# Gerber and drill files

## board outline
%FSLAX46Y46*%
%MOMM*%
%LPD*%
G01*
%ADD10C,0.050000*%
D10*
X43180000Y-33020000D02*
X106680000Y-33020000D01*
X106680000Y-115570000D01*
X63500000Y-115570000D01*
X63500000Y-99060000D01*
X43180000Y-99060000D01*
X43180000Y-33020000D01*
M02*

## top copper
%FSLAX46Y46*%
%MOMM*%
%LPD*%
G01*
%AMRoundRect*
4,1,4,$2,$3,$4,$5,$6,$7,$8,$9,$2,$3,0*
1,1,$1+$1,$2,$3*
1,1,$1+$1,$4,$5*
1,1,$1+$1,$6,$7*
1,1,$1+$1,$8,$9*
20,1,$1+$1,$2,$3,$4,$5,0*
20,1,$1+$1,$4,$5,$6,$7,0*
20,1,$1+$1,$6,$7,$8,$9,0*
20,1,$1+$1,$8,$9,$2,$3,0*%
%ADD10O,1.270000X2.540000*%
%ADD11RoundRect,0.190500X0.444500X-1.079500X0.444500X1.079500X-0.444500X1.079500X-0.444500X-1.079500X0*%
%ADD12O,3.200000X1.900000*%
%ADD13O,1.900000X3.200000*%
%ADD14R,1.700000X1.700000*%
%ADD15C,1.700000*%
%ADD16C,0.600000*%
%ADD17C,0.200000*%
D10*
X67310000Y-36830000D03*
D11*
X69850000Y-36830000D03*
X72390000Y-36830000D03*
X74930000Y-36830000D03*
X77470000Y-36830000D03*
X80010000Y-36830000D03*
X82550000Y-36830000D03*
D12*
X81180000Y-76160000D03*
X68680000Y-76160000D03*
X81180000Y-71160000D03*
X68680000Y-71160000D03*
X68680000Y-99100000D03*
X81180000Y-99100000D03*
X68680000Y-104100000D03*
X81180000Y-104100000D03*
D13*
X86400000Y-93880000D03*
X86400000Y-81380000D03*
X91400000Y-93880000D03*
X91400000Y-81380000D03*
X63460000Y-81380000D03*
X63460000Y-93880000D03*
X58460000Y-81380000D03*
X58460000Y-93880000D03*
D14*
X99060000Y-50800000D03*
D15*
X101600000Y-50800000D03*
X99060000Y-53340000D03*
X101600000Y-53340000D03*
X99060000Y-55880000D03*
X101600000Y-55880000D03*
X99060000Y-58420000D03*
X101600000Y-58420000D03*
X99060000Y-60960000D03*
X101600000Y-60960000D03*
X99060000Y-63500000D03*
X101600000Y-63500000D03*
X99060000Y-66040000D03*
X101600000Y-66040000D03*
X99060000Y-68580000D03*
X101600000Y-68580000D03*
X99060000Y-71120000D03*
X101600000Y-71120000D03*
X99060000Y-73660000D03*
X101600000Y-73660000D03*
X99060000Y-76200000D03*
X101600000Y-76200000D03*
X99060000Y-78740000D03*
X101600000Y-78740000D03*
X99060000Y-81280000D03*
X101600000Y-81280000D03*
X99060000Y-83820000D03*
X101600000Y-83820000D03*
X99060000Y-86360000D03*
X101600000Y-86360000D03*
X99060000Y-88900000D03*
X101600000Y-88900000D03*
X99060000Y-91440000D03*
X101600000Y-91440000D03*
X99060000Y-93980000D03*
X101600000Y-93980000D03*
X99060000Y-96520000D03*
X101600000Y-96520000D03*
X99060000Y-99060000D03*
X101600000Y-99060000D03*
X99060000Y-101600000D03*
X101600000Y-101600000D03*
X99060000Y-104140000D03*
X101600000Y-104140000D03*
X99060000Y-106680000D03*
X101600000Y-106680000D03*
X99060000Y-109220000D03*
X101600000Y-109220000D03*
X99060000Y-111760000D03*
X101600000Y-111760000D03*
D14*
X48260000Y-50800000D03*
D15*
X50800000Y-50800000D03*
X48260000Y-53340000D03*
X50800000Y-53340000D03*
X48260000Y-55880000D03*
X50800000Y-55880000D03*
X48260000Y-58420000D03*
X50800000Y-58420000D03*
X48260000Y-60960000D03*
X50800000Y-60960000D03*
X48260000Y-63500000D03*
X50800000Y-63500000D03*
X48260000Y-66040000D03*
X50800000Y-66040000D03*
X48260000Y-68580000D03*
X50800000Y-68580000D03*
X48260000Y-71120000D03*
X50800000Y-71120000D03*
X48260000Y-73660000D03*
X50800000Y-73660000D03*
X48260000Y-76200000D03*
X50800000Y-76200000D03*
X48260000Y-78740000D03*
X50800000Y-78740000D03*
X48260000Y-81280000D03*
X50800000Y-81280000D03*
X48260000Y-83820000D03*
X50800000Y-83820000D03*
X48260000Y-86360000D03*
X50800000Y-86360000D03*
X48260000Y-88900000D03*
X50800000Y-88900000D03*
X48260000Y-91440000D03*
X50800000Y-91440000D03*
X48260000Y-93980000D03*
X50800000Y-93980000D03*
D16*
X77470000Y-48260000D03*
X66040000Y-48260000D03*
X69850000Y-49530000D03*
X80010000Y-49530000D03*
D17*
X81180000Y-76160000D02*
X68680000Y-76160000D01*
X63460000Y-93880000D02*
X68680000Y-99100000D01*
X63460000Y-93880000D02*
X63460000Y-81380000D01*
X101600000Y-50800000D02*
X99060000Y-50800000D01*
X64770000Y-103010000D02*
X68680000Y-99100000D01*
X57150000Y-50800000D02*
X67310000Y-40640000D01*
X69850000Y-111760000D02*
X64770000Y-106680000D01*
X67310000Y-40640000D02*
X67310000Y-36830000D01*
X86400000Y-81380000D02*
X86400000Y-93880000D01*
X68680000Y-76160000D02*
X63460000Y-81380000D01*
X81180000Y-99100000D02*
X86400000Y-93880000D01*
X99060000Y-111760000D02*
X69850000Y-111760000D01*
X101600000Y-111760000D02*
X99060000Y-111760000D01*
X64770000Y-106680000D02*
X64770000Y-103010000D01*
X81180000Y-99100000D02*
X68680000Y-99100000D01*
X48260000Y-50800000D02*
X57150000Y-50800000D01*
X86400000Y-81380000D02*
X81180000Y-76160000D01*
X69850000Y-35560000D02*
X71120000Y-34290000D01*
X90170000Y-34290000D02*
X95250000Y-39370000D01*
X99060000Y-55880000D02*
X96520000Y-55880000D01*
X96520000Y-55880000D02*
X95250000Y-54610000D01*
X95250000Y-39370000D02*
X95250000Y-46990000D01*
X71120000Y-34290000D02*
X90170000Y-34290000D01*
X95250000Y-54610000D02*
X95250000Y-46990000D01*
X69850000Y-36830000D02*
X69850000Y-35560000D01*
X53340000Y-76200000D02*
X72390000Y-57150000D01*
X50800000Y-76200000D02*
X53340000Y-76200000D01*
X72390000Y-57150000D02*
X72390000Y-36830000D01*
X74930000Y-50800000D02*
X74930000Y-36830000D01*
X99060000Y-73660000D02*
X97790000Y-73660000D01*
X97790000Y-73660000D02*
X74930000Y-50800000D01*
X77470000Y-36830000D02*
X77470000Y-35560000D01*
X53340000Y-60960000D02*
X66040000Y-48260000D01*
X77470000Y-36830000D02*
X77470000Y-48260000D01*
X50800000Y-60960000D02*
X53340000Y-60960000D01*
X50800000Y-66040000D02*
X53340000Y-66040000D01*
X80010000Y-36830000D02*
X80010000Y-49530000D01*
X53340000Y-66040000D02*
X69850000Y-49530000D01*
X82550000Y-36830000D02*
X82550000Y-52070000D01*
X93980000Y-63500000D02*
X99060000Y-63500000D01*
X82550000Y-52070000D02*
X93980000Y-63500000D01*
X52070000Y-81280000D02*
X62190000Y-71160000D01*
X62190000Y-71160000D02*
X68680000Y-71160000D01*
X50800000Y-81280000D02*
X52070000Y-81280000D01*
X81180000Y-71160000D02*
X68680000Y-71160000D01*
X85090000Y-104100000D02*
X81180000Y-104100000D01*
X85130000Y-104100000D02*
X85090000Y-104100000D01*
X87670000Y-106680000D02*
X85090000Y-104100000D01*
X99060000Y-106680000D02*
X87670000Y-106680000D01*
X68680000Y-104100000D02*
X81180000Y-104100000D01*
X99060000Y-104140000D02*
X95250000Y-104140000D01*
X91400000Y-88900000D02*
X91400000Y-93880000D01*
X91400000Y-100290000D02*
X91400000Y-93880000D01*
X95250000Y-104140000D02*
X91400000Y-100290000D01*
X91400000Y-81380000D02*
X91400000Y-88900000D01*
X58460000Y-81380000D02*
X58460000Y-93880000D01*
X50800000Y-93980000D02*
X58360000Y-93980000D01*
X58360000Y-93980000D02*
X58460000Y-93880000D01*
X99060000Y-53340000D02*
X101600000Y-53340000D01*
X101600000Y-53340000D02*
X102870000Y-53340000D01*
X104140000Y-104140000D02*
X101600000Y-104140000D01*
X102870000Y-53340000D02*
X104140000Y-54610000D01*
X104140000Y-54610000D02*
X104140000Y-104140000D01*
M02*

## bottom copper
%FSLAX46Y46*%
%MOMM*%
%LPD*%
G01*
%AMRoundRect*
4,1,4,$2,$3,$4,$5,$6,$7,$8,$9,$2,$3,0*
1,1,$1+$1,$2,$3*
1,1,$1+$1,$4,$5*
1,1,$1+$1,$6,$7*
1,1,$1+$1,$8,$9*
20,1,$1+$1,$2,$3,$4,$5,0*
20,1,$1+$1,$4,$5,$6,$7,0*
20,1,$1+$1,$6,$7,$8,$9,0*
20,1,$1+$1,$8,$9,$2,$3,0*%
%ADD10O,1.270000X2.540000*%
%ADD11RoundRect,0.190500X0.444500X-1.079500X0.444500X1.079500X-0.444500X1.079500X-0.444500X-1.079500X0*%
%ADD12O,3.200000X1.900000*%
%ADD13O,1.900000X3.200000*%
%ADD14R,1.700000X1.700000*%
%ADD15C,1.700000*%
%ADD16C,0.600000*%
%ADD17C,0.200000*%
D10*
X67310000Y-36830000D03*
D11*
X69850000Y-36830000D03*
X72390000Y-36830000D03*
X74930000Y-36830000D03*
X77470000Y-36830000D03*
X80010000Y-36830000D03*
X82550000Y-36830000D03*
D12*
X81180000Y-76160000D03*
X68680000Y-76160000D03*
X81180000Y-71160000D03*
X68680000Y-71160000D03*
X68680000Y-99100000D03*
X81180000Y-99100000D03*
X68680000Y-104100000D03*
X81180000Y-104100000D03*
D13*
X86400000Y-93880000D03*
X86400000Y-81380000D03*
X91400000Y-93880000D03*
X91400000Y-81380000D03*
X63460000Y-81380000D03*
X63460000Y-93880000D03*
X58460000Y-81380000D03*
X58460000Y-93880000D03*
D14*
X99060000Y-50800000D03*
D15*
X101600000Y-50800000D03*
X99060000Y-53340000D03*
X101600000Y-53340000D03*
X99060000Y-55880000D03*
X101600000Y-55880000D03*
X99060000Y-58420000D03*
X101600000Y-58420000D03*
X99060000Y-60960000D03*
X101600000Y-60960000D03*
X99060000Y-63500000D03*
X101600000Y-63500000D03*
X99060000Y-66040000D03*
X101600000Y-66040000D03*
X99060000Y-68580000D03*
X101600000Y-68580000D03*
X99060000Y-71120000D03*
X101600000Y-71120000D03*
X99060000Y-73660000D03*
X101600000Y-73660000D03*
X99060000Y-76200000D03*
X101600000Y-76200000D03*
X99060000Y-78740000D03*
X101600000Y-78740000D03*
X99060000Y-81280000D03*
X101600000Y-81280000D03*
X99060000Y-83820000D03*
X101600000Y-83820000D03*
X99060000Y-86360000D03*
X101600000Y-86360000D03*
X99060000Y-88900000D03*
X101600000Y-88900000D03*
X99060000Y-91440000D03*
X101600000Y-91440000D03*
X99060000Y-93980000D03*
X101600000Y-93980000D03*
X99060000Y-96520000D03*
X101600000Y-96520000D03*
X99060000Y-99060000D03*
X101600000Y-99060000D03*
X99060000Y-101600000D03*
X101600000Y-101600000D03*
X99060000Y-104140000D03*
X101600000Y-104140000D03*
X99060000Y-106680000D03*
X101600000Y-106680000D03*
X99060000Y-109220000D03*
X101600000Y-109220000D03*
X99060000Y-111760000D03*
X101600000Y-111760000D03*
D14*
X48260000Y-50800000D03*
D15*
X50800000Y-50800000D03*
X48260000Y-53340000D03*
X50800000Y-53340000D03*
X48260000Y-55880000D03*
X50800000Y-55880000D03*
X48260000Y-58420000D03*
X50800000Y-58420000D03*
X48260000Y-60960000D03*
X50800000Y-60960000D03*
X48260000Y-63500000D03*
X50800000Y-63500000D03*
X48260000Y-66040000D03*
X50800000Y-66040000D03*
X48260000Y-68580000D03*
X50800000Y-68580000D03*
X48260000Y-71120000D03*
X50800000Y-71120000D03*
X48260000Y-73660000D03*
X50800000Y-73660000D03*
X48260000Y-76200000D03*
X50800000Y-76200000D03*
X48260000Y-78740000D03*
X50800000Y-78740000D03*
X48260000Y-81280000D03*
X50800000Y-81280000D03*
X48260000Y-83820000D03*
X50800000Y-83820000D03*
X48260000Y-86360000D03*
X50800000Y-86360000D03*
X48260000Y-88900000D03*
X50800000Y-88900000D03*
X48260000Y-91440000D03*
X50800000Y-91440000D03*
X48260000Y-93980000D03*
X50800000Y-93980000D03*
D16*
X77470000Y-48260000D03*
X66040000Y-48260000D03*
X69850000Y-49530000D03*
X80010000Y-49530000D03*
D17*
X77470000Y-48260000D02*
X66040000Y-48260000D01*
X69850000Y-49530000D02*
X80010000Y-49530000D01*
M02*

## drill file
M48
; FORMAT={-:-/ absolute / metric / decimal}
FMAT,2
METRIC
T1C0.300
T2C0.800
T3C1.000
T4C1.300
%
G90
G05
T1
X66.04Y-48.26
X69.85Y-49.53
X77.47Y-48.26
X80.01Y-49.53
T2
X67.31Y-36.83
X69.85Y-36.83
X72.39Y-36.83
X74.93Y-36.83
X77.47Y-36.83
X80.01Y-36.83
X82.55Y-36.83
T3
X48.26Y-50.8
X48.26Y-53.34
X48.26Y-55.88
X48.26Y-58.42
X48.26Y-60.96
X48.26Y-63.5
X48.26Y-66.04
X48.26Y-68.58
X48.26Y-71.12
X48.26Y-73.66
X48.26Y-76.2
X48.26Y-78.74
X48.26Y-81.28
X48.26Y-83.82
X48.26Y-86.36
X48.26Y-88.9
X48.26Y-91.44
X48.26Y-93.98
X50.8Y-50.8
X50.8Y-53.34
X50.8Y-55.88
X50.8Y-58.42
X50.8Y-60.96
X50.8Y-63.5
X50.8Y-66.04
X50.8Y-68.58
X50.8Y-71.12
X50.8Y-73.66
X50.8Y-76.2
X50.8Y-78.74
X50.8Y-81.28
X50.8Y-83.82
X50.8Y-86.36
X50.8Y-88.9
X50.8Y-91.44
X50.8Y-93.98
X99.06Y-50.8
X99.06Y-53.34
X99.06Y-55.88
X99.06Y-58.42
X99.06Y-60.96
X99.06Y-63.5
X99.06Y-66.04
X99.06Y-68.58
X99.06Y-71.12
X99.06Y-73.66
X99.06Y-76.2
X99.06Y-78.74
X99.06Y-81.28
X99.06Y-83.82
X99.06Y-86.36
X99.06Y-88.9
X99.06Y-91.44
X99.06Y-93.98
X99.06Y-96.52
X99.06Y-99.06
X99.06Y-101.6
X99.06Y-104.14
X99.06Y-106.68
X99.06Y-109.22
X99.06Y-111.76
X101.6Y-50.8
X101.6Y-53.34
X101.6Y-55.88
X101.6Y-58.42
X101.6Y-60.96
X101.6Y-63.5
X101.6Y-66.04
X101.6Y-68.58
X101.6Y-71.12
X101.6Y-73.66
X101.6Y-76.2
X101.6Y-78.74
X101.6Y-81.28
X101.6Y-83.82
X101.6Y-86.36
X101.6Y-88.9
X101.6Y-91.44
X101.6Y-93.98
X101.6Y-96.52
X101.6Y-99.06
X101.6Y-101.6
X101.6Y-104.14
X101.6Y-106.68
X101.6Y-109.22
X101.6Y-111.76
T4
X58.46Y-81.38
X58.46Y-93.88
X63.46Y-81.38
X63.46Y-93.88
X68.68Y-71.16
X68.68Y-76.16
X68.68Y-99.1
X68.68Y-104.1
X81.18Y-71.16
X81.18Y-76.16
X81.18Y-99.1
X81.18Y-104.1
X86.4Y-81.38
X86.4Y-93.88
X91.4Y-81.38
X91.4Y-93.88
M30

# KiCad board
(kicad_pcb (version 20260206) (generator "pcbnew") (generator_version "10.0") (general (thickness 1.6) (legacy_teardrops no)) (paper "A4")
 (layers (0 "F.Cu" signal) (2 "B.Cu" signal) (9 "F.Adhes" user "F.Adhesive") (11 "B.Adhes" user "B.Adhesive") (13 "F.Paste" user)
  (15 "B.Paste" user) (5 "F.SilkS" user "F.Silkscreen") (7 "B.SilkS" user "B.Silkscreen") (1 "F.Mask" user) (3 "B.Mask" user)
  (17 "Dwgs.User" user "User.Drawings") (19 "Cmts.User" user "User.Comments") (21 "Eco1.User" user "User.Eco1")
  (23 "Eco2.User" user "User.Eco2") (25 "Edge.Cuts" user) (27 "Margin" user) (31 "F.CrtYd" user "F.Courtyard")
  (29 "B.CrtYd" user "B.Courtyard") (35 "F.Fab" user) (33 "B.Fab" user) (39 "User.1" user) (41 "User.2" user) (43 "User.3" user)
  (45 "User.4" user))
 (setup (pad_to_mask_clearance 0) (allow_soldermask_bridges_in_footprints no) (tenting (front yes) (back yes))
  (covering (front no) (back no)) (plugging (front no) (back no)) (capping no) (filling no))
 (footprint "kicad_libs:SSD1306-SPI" (layer "F.Cu") (at 74.93 46.99)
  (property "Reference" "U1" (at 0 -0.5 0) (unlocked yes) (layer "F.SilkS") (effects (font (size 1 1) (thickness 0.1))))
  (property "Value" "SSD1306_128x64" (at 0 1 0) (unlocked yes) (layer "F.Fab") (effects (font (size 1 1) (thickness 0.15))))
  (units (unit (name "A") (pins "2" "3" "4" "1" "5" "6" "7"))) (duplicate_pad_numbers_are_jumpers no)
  (pad "1" thru_hole oval (at -7.62 -10.16 90) (size 2.54 1.27) (drill 0.8) (layers "*.Cu" "*.Mask") (remove_unused_layers no) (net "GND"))
  (pad "2" thru_hole roundrect (at -5.08 -10.16 90) (size 2.54 1.27) (drill 0.8) (layers "*.Cu" "*.Mask") (remove_unused_layers no)
   (roundrect_rratio 0.15) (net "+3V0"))
  (pad "3" thru_hole roundrect (at -2.54 -10.16 90) (size 2.54 1.27) (drill 0.8) (layers "*.Cu" "*.Mask") (remove_unused_layers no)
   (roundrect_rratio 0.15) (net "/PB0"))
  (pad "4" thru_hole roundrect (at 0 -10.16 90) (size 2.54 1.27) (drill 0.8) (layers "*.Cu" "*.Mask") (remove_unused_layers no)
   (roundrect_rratio 0.15) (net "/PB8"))
  (pad "5" thru_hole roundrect (at 2.54 -10.16 90) (size 2.54 1.27) (drill 0.8) (layers "*.Cu" "*.Mask") (remove_unused_layers no)
   (roundrect_rratio 0.15) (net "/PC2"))
  (pad "6" thru_hole roundrect (at 5.08 -10.16 90) (size 2.54 1.27) (drill 0.8) (layers "*.Cu" "*.Mask") (remove_unused_layers no)
   (roundrect_rratio 0.15) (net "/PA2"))
  (pad "7" thru_hole roundrect (at 7.62 -10.16 90) (size 2.54 1.27) (drill 0.8) (layers "*.Cu" "*.Mask") (remove_unused_layers no)
   (roundrect_rratio 0.15) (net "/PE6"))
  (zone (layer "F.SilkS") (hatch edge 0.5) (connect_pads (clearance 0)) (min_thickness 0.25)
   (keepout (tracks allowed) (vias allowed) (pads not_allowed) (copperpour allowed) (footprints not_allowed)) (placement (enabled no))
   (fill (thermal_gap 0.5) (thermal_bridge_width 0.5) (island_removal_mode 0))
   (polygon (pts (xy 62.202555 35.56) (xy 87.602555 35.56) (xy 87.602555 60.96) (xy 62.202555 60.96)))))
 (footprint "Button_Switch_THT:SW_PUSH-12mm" (layer "F.Cu") (at 81.18 76.16 180)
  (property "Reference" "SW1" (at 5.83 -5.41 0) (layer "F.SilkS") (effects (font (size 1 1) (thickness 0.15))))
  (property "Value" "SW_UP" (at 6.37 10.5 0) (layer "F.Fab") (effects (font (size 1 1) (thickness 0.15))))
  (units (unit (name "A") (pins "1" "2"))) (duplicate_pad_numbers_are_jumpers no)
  (pad "1" thru_hole oval (at 0 0 180) (size 3.2 1.9) (drill 1.3) (layers "*.Cu" "*.Mask") (remove_unused_layers no) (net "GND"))
  (pad "1" thru_hole oval (at 12.5 0 180) (size 3.2 1.9) (drill 1.3) (layers "*.Cu" "*.Mask") (remove_unused_layers no) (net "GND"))
  (pad "2" thru_hole oval (at 0 5 180) (size 3.2 1.9) (drill 1.3) (layers "*.Cu" "*.Mask") (remove_unused_layers no) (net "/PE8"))
  (pad "2" thru_hole oval (at 12.5 5 180) (size 3.2 1.9) (drill 1.3) (layers "*.Cu" "*.Mask") (remove_unused_layers no) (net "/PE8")))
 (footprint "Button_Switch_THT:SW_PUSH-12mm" (layer "F.Cu") (at 68.68 99.1)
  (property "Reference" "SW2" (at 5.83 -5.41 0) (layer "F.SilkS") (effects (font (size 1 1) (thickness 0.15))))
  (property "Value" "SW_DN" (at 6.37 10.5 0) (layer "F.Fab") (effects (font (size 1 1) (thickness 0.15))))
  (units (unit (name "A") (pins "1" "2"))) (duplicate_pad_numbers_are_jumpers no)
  (pad "1" thru_hole oval (at 0 0) (size 3.2 1.9) (drill 1.3) (layers "*.Cu" "*.Mask") (remove_unused_layers no) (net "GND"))
  (pad "1" thru_hole oval (at 12.5 0) (size 3.2 1.9) (drill 1.3) (layers "*.Cu" "*.Mask") (remove_unused_layers no) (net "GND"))
  (pad "2" thru_hole oval (at 0 5) (size 3.2 1.9) (drill 1.3) (layers "*.Cu" "*.Mask") (remove_unused_layers no) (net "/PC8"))
  (pad "2" thru_hole oval (at 12.5 5) (size 3.2 1.9) (drill 1.3) (layers "*.Cu" "*.Mask") (remove_unused_layers no) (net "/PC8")))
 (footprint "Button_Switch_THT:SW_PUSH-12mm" (layer "F.Cu") (at 86.4 93.88 90)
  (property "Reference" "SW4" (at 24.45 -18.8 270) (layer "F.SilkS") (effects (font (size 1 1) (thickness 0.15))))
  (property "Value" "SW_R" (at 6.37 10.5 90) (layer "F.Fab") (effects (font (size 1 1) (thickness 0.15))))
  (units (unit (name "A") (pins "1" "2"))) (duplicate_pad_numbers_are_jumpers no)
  (pad "1" thru_hole oval (at 0 0 90) (size 3.2 1.9) (drill 1.3) (layers "*.Cu" "*.Mask") (remove_unused_layers no) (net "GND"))
  (pad "1" thru_hole oval (at 12.5 0 90) (size 3.2 1.9) (drill 1.3) (layers "*.Cu" "*.Mask") (remove_unused_layers no) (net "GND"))
  (pad "2" thru_hole oval (at 0 5 90) (size 3.2 1.9) (drill 1.3) (layers "*.Cu" "*.Mask") (remove_unused_layers no) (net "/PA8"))
  (pad "2" thru_hole oval (at 12.5 5 90) (size 3.2 1.9) (drill 1.3) (layers "*.Cu" "*.Mask") (remove_unused_layers no) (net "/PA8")))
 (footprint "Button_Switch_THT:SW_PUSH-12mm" (layer "F.Cu") (at 63.46 81.38 -90)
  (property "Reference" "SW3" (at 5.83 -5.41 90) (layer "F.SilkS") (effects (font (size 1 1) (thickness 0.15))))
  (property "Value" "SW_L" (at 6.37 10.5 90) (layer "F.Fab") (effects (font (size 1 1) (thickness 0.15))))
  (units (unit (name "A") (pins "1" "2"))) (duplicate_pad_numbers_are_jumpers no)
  (pad "1" thru_hole oval (at 0 0 270) (size 3.2 1.9) (drill 1.3) (layers "*.Cu" "*.Mask") (remove_unused_layers no) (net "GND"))
  (pad "1" thru_hole oval (at 12.5 0 270) (size 3.2 1.9) (drill 1.3) (layers "*.Cu" "*.Mask") (remove_unused_layers no) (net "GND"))
  (pad "2" thru_hole oval (at 0 5 270) (size 3.2 1.9) (drill 1.3) (layers "*.Cu" "*.Mask") (remove_unused_layers no) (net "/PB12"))
  (pad "2" thru_hole oval (at 12.5 5 270) (size 3.2 1.9) (drill 1.3) (layers "*.Cu" "*.Mask") (remove_unused_layers no) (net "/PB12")))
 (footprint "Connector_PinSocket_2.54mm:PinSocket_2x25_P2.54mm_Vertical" (layer "B.Cu") (at 99.06 50.8 180)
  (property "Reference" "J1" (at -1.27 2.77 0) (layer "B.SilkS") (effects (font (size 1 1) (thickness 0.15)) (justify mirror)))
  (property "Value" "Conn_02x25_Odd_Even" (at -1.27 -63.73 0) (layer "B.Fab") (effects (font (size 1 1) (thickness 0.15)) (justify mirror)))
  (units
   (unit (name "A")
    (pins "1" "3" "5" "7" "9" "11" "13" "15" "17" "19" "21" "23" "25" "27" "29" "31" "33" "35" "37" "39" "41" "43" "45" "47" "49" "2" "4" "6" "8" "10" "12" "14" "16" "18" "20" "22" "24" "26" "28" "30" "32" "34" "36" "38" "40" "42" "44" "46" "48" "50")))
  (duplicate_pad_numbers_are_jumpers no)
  (pad "1" thru_hole rect (at 0 0 180) (size 1.7 1.7) (drill 1) (layers "*.Cu" "*.Mask") (remove_unused_layers no) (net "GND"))
  (pad "2" thru_hole circle (at -2.54 0 180) (size 1.7 1.7) (drill 1) (layers "*.Cu" "*.Mask") (remove_unused_layers no) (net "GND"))
  (pad "3" thru_hole circle (at 0 -2.54 180) (size 1.7 1.7) (drill 1) (layers "*.Cu" "*.Mask") (remove_unused_layers no) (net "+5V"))
  (pad "4" thru_hole circle (at -2.54 -2.54 180) (size 1.7 1.7) (drill 1) (layers "*.Cu" "*.Mask") (remove_unused_layers no) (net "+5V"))
  (pad "5" thru_hole circle (at 0 -5.08 180) (size 1.7 1.7) (drill 1) (layers "*.Cu" "*.Mask") (remove_unused_layers no) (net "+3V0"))
  (pad "6" thru_hole circle (at -2.54 -5.08 180) (size 1.7 1.7) (drill 1) (layers "*.Cu" "*.Mask") (remove_unused_layers no) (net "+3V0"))
  (pad "7" thru_hole circle (at 0 -7.62 180) (size 1.7 1.7) (drill 1) (layers "*.Cu" "*.Mask") (remove_unused_layers no)
   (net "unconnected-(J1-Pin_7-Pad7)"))
  (pad "8" thru_hole circle (at -2.54 -7.62 180) (size 1.7 1.7) (drill 1) (layers "*.Cu" "*.Mask") (remove_unused_layers no)
   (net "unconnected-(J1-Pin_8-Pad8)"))
  (pad "9" thru_hole circle (at 0 -10.16 180) (size 1.7 1.7) (drill 1) (layers "*.Cu" "*.Mask") (remove_unused_layers no)
   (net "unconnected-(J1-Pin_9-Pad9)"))
  (pad "10" thru_hole circle (at -2.54 -10.16 180) (size 1.7 1.7) (drill 1) (layers "*.Cu" "*.Mask") (remove_unused_layers no)
   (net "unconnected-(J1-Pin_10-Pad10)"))
  (pad "11" thru_hole circle (at 0 -12.7 180) (size 1.7 1.7) (drill 1) (layers "*.Cu" "*.Mask") (remove_unused_layers no) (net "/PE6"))
  (pad "12" thru_hole circle (at -2.54 -12.7 180) (size 1.7 1.7) (drill 1) (layers "*.Cu" "*.Mask") (remove_unused_layers no)
   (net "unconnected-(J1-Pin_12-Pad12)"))
  (pad "13" thru_hole circle (at 0 -15.24 180) (size 1.7 1.7) (drill 1) (layers "*.Cu" "*.Mask") (remove_unused_layers no)
   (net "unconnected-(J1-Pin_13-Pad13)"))
  (pad "14" thru_hole circle (at -2.54 -15.24 180) (size 1.7 1.7) (drill 1) (layers "*.Cu" "*.Mask") (remove_unused_layers no)
   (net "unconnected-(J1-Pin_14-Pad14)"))
  (pad "15" thru_hole circle (at 0 -17.78 180) (size 1.7 1.7) (drill 1) (layers "*.Cu" "*.Mask") (remove_unused_layers no)
   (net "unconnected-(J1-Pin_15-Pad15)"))
  (pad "16" thru_hole circle (at -2.54 -17.78 180) (size 1.7 1.7) (drill 1) (layers "*.Cu" "*.Mask") (remove_unused_layers no)
   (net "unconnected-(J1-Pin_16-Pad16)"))
  (pad "17" thru_hole circle (at 0 -20.32 180) (size 1.7 1.7) (drill 1) (layers "*.Cu" "*.Mask") (remove_unused_layers no) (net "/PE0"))
  (pad "18" thru_hole circle (at -2.54 -20.32 180) (size 1.7 1.7) (drill 1) (layers "*.Cu" "*.Mask") (remove_unused_layers no)
   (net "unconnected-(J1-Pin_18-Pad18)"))
  (pad "19" thru_hole circle (at 0 -22.86 180) (size 1.7 1.7) (drill 1) (layers "*.Cu" "*.Mask") (remove_unused_layers no) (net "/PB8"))
  (pad "20" thru_hole circle (at -2.54 -22.86 180) (size 1.7 1.7) (drill 1) (layers "*.Cu" "*.Mask") (remove_unused_layers no)
   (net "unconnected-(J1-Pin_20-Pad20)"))
  (pad "21" thru_hole circle (at 0 -25.4 180) (size 1.7 1.7) (drill 1) (layers "*.Cu" "*.Mask") (remove_unused_layers no)
   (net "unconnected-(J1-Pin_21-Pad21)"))
  (pad "22" thru_hole circle (at -2.54 -25.4 180) (size 1.7 1.7) (drill 1) (layers "*.Cu" "*.Mask") (remove_unused_layers no)
   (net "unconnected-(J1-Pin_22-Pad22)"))
  (pad "23" thru_hole circle (at 0 -27.94 180) (size 1.7 1.7) (drill 1) (layers "*.Cu" "*.Mask") (remove_unused_layers no)
   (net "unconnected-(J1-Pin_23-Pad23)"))
  (pad "24" thru_hole circle (at -2.54 -27.94 180) (size 1.7 1.7) (drill 1) (layers "*.Cu" "*.Mask") (remove_unused_layers no)
   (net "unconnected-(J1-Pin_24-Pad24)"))
  (pad "25" thru_hole circle (at 0 -30.48 180) (size 1.7 1.7) (drill 1) (layers "*.Cu" "*.Mask") (remove_unused_layers no)
   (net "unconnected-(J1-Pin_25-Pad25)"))
  (pad "26" thru_hole circle (at -2.54 -30.48 180) (size 1.7 1.7) (drill 1) (layers "*.Cu" "*.Mask") (remove_unused_layers no)
   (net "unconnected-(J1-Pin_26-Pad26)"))
  (pad "27" thru_hole circle (at 0 -33.02 180) (size 1.7 1.7) (drill 1) (layers "*.Cu" "*.Mask") (remove_unused_layers no)
   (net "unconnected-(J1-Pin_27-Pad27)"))
  (pad "28" thru_hole circle (at -2.54 -33.02 180) (size 1.7 1.7) (drill 1) (layers "*.Cu" "*.Mask") (remove_unused_layers no)
   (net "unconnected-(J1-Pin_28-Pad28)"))
  (pad "29" thru_hole circle (at 0 -35.56 180) (size 1.7 1.7) (drill 1) (layers "*.Cu" "*.Mask") (remove_unused_layers no)
   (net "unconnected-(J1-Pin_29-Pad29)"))
  (pad "30" thru_hole circle (at -2.54 -35.56 180) (size 1.7 1.7) (drill 1) (layers "*.Cu" "*.Mask") (remove_unused_layers no)
   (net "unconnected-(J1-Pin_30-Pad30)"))
  (pad "31" thru_hole circle (at 0 -38.1 180) (size 1.7 1.7) (drill 1) (layers "*.Cu" "*.Mask") (remove_unused_layers no) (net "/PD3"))
  (pad "32" thru_hole circle (at -2.54 -38.1 180) (size 1.7 1.7) (drill 1) (layers "*.Cu" "*.Mask") (remove_unused_layers no)
   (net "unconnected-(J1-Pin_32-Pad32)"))
  (pad "33" thru_hole circle (at 0 -40.64 180) (size 1.7 1.7) (drill 1) (layers "*.Cu" "*.Mask") (remove_unused_layers no) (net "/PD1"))
  (pad "34" thru_hole circle (at -2.54 -40.64 180) (size 1.7 1.7) (drill 1) (layers "*.Cu" "*.Mask") (remove_unused_layers no)
   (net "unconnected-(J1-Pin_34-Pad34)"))
  (pad "35" thru_hole circle (at 0 -43.18 180) (size 1.7 1.7) (drill 1) (layers "*.Cu" "*.Mask") (remove_unused_layers no)
   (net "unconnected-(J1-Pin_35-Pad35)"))
  (pad "36" thru_hole circle (at -2.54 -43.18 180) (size 1.7 1.7) (drill 1) (layers "*.Cu" "*.Mask") (remove_unused_layers no)
   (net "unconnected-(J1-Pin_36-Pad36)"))
  (pad "37" thru_hole circle (at 0 -45.72 180) (size 1.7 1.7) (drill 1) (layers "*.Cu" "*.Mask") (remove_unused_layers no)
   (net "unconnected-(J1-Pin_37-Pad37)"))
  (pad "38" thru_hole circle (at -2.54 -45.72 180) (size 1.7 1.7) (drill 1) (layers "*.Cu" "*.Mask") (remove_unused_layers no)
   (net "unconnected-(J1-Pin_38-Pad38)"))
  (pad "39" thru_hole circle (at 0 -48.26 180) (size 1.7 1.7) (drill 1) (layers "*.Cu" "*.Mask") (remove_unused_layers no)
   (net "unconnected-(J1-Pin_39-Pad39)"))
  (pad "40" thru_hole circle (at -2.54 -48.26 180) (size 1.7 1.7) (drill 1) (layers "*.Cu" "*.Mask") (remove_unused_layers no)
   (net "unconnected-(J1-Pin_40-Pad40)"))
  (pad "41" thru_hole circle (at 0 -50.8 180) (size 1.7 1.7) (drill 1) (layers "*.Cu" "*.Mask") (remove_unused_layers no)
   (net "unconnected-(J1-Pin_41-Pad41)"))
  (pad "42" thru_hole circle (at -2.54 -50.8 180) (size 1.7 1.7) (drill 1) (layers "*.Cu" "*.Mask") (remove_unused_layers no)
   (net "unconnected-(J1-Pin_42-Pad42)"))
  (pad "43" thru_hole circle (at 0 -53.34 180) (size 1.7 1.7) (drill 1) (layers "*.Cu" "*.Mask") (remove_unused_layers no) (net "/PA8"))
  (pad "44" thru_hole circle (at -2.54 -53.34 180) (size 1.7 1.7) (drill 1) (layers "*.Cu" "*.Mask") (remove_unused_layers no) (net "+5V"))
  (pad "45" thru_hole circle (at 0 -55.88 180) (size 1.7 1.7) (drill 1) (layers "*.Cu" "*.Mask") (remove_unused_layers no) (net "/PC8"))
  (pad "46" thru_hole circle (at -2.54 -55.88 180) (size 1.7 1.7) (drill 1) (layers "*.Cu" "*.Mask") (remove_unused_layers no)
   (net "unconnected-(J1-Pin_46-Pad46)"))
  (pad "47" thru_hole circle (at 0 -58.42 180) (size 1.7 1.7) (drill 1) (layers "*.Cu" "*.Mask") (remove_unused_layers no)
   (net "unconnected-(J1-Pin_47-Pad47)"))
  (pad "48" thru_hole circle (at -2.54 -58.42 180) (size 1.7 1.7) (drill 1) (layers "*.Cu" "*.Mask") (remove_unused_layers no)
   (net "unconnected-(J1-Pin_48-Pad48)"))
  (pad "49" thru_hole circle (at 0 -60.96 180) (size 1.7 1.7) (drill 1) (layers "*.Cu" "*.Mask") (remove_unused_layers no) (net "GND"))
  (pad "50" thru_hole circle (at -2.54 -60.96 180) (size 1.7 1.7) (drill 1) (layers "*.Cu" "*.Mask") (remove_unused_layers no) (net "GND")))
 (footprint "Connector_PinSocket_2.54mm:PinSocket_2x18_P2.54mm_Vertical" (layer "B.Cu") (at 48.26 50.8 180)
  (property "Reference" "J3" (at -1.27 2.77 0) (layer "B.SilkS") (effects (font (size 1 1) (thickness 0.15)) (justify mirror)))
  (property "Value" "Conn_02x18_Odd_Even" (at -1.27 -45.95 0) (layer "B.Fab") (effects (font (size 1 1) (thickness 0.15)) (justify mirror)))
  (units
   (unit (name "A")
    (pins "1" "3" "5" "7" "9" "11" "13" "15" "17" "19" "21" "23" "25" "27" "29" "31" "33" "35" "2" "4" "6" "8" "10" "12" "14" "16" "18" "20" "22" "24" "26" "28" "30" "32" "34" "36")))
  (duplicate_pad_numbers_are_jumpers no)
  (pad "1" thru_hole rect (at 0 0 180) (size 1.7 1.7) (drill 1) (layers "*.Cu" "*.Mask") (remove_unused_layers no) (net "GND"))
  (pad "2" thru_hole circle (at -2.54 0 180) (size 1.7 1.7) (drill 1) (layers "*.Cu" "*.Mask") (remove_unused_layers no) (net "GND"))
  (pad "3" thru_hole circle (at 0 -2.54 180) (size 1.7 1.7) (drill 1) (layers "*.Cu" "*.Mask") (remove_unused_layers no) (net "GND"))
  (pad "4" thru_hole circle (at -2.54 -2.54 180) (size 1.7 1.7) (drill 1) (layers "*.Cu" "*.Mask") (remove_unused_layers no)
   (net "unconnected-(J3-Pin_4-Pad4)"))
  (pad "5" thru_hole circle (at 0 -5.08 180) (size 1.7 1.7) (drill 1) (layers "*.Cu" "*.Mask") (remove_unused_layers no)
   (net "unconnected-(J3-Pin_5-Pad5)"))
  (pad "6" thru_hole circle (at -2.54 -5.08 180) (size 1.7 1.7) (drill 1) (layers "*.Cu" "*.Mask") (remove_unused_layers no)
   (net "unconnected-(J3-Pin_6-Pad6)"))
  (pad "7" thru_hole circle (at 0 -7.62 180) (size 1.7 1.7) (drill 1) (layers "*.Cu" "*.Mask") (remove_unused_layers no)
   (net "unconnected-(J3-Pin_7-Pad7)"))
  (pad "8" thru_hole circle (at -2.54 -7.62 180) (size 1.7 1.7) (drill 1) (layers "*.Cu" "*.Mask") (remove_unused_layers no)
   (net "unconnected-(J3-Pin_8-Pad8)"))
  (pad "9" thru_hole circle (at 0 -10.16 180) (size 1.7 1.7) (drill 1) (layers "*.Cu" "*.Mask") (remove_unused_layers no)
   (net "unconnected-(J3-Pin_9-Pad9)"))
  (pad "10" thru_hole circle (at -2.54 -10.16 180) (size 1.7 1.7) (drill 1) (layers "*.Cu" "*.Mask") (remove_unused_layers no) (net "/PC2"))
  (pad "11" thru_hole circle (at 0 -12.7 180) (size 1.7 1.7) (drill 1) (layers "*.Cu" "*.Mask") (remove_unused_layers no)
   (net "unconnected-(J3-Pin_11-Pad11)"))
  (pad "12" thru_hole circle (at -2.54 -12.7 180) (size 1.7 1.7) (drill 1) (layers "*.Cu" "*.Mask") (remove_unused_layers no)
   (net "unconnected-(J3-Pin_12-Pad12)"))
  (pad "13" thru_hole circle (at 0 -15.24 180) (size 1.7 1.7) (drill 1) (layers "*.Cu" "*.Mask") (remove_unused_layers no)
   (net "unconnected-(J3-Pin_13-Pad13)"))
  (pad "14" thru_hole circle (at -2.54 -15.24 180) (size 1.7 1.7) (drill 1) (layers "*.Cu" "*.Mask") (remove_unused_layers no) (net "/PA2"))
  (pad "15" thru_hole circle (at 0 -17.78 180) (size 1.7 1.7) (drill 1) (layers "*.Cu" "*.Mask") (remove_unused_layers no)
   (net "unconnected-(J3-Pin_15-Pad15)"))
  (pad "16" thru_hole circle (at -2.54 -17.78 180) (size 1.7 1.7) (drill 1) (layers "*.Cu" "*.Mask") (remove_unused_layers no)
   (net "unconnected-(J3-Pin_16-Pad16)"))
  (pad "17" thru_hole circle (at 0 -20.32 180) (size 1.7 1.7) (drill 1) (layers "*.Cu" "*.Mask") (remove_unused_layers no)
   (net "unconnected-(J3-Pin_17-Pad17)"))
  (pad "18" thru_hole circle (at -2.54 -20.32 180) (size 1.7 1.7) (drill 1) (layers "*.Cu" "*.Mask") (remove_unused_layers no)
   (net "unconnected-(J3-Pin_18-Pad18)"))
  (pad "19" thru_hole circle (at 0 -22.86 180) (size 1.7 1.7) (drill 1) (layers "*.Cu" "*.Mask") (remove_unused_layers no)
   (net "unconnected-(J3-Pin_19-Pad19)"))
  (pad "20" thru_hole circle (at -2.54 -22.86 180) (size 1.7 1.7) (drill 1) (layers "*.Cu" "*.Mask") (remove_unused_layers no)
   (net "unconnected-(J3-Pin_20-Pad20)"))
  (pad "21" thru_hole circle (at 0 -25.4 180) (size 1.7 1.7) (drill 1) (layers "*.Cu" "*.Mask") (remove_unused_layers no)
   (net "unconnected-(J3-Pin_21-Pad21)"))
  (pad "22" thru_hole circle (at -2.54 -25.4 180) (size 1.7 1.7) (drill 1) (layers "*.Cu" "*.Mask") (remove_unused_layers no) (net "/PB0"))
  (pad "23" thru_hole circle (at 0 -27.94 180) (size 1.7 1.7) (drill 1) (layers "*.Cu" "*.Mask") (remove_unused_layers no) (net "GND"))
  (pad "24" thru_hole circle (at -2.54 -27.94 180) (size 1.7 1.7) (drill 1) (layers "*.Cu" "*.Mask") (remove_unused_layers no)
   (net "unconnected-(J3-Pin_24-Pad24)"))
  (pad "25" thru_hole circle (at 0 -30.48 180) (size 1.7 1.7) (drill 1) (layers "*.Cu" "*.Mask") (remove_unused_layers no)
   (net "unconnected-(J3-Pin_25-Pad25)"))
  (pad "26" thru_hole circle (at -2.54 -30.48 180) (size 1.7 1.7) (drill 1) (layers "*.Cu" "*.Mask") (remove_unused_layers no) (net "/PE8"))
  (pad "27" thru_hole circle (at 0 -33.02 180) (size 1.7 1.7) (drill 1) (layers "*.Cu" "*.Mask") (remove_unused_layers no)
   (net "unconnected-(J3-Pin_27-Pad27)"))
  (pad "28" thru_hole circle (at -2.54 -33.02 180) (size 1.7 1.7) (drill 1) (layers "*.Cu" "*.Mask") (remove_unused_layers no)
   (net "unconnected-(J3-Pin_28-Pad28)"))
  (pad "29" thru_hole circle (at 0 -35.56 180) (size 1.7 1.7) (drill 1) (layers "*.Cu" "*.Mask") (remove_unused_layers no)
   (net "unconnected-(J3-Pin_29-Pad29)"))
  (pad "30" thru_hole circle (at -2.54 -35.56 180) (size 1.7 1.7) (drill 1) (layers "*.Cu" "*.Mask") (remove_unused_layers no) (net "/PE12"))
  (pad "31" thru_hole circle (at 0 -38.1 180) (size 1.7 1.7) (drill 1) (layers "*.Cu" "*.Mask") (remove_unused_layers no)
   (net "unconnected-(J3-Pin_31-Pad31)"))
  (pad "32" thru_hole circle (at -2.54 -38.1 180) (size 1.7 1.7) (drill 1) (layers "*.Cu" "*.Mask") (remove_unused_layers no) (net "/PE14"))
  (pad "33" thru_hole circle (at 0 -40.64 180) (size 1.7 1.7) (drill 1) (layers "*.Cu" "*.Mask") (remove_unused_layers no) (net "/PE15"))
  (pad "34" thru_hole circle (at -2.54 -40.64 180) (size 1.7 1.7) (drill 1) (layers "*.Cu" "*.Mask") (remove_unused_layers no)
   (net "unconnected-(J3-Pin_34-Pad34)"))
  (pad "35" thru_hole circle (at 0 -43.18 180) (size 1.7 1.7) (drill 1) (layers "*.Cu" "*.Mask") (remove_unused_layers no)
   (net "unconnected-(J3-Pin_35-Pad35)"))
  (pad "36" thru_hole circle (at -2.54 -43.18 180) (size 1.7 1.7) (drill 1) (layers "*.Cu" "*.Mask") (remove_unused_layers no) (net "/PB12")))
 (gr_poly
  (pts (xy 43.18 33.02) (xy 106.68 33.02) (xy 106.68 115.57) (xy 63.5 115.57) (xy 63.5 99.06) (xy 43.18 99.06))
  (stroke (width 0.05) (type solid)) (fill no) (layer "Edge.Cuts"))
 (segment (start 81.18 76.16) (end 68.68 76.16) (width 0.2) (layer "F.Cu") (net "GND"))
 (segment (start 63.46 93.88) (end 68.68 99.1) (width 0.2) (layer "F.Cu") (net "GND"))
 (segment (start 63.46 93.88) (end 63.46 81.38) (width 0.2) (layer "F.Cu") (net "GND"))
 (segment (start 101.6 50.8) (end 99.06 50.8) (width 0.2) (layer "F.Cu") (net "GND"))
 (segment (start 64.77 103.01) (end 68.68 99.1) (width 0.2) (layer "F.Cu") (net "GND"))
 (segment (start 57.15 50.8) (end 67.31 40.64) (width 0.2) (layer "F.Cu") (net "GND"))
 (segment (start 69.85 111.76) (end 64.77 106.68) (width 0.2) (layer "F.Cu") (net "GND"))
 (segment (start 67.31 40.64) (end 67.31 36.83) (width 0.2) (layer "F.Cu") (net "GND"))
 (segment (start 86.4 81.38) (end 86.4 93.88) (width 0.2) (layer "F.Cu") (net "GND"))
 (segment (start 68.68 76.16) (end 63.46 81.38) (width 0.2) (layer "F.Cu") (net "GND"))
 (segment (start 81.18 99.1) (end 86.4 93.88) (width 0.2) (layer "F.Cu") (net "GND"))
 (segment (start 99.06 111.76) (end 69.85 111.76) (width 0.2) (layer "F.Cu") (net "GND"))
 (segment (start 101.6 111.76) (end 99.06 111.76) (width 0.2) (layer "F.Cu") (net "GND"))
 (segment (start 64.77 106.68) (end 64.77 103.01) (width 0.2) (layer "F.Cu") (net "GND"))
 (segment (start 81.18 99.1) (end 68.68 99.1) (width 0.2) (layer "F.Cu") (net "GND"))
 (segment (start 48.26 50.8) (end 57.15 50.8) (width 0.2) (layer "F.Cu") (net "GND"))
 (segment (start 86.4 81.38) (end 81.18 76.16) (width 0.2) (layer "F.Cu") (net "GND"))
 (segment (start 69.85 35.56) (end 71.12 34.29) (width 0.2) (layer "F.Cu") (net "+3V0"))
 (segment (start 90.17 34.29) (end 95.25 39.37) (width 0.2) (layer "F.Cu") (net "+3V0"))
 (segment (start 99.06 55.88) (end 96.52 55.88) (width 0.2) (layer "F.Cu") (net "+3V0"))
 (segment (start 96.52 55.88) (end 95.25 54.61) (width 0.2) (layer "F.Cu") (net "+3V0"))
 (segment (start 95.25 39.37) (end 95.25 46.99) (width 0.2) (layer "F.Cu") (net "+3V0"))
 (segment (start 71.12 34.29) (end 90.17 34.29) (width 0.2) (layer "F.Cu") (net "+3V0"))
 (segment (start 95.25 54.61) (end 95.25 46.99) (width 0.2) (layer "F.Cu") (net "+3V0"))
 (segment (start 69.85 36.83) (end 69.85 35.56) (width 0.2) (layer "F.Cu") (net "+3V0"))
 (segment (start 53.34 76.2) (end 72.39 57.15) (width 0.2) (layer "F.Cu") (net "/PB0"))
 (segment (start 50.8 76.2) (end 53.34 76.2) (width 0.2) (layer "F.Cu") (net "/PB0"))
 (segment (start 72.39 57.15) (end 72.39 36.83) (width 0.2) (layer "F.Cu") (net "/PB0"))
 (segment (start 74.93 50.8) (end 74.93 36.83) (width 0.2) (layer "F.Cu") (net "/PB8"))
 (segment (start 99.06 73.66) (end 97.79 73.66) (width 0.2) (layer "F.Cu") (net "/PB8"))
 (segment (start 97.79 73.66) (end 74.93 50.8) (width 0.2) (layer "F.Cu") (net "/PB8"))
 (segment (start 77.47 36.83) (end 77.47 35.56) (width 0.2) (layer "F.Cu") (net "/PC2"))
 (segment (start 53.34 60.96) (end 66.04 48.26) (width 0.2) (layer "F.Cu") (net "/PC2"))
 (segment (start 77.47 36.83) (end 77.47 48.26) (width 0.2) (layer "F.Cu") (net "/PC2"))
 (segment (start 50.8 60.96) (end 53.34 60.96) (width 0.2) (layer "F.Cu") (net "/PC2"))
 (via (at 77.47 48.26) (size 0.6) (drill 0.3) (layers "F.Cu" "B.Cu") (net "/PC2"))
 (via (at 66.04 48.26) (size 0.6) (drill 0.3) (layers "F.Cu" "B.Cu") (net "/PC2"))
 (segment (start 77.47 48.26) (end 66.04 48.26) (width 0.2) (layer "B.Cu") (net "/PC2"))
 (segment (start 50.8 66.04) (end 53.34 66.04) (width 0.2) (layer "F.Cu") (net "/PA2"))
 (segment (start 80.01 36.83) (end 80.01 49.53) (width 0.2) (layer "F.Cu") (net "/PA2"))
 (segment (start 53.34 66.04) (end 69.85 49.53) (width 0.2) (layer "F.Cu") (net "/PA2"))
 (via (at 69.85 49.53) (size 0.6) (drill 0.3) (layers "F.Cu" "B.Cu") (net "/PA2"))
 (via (at 80.01 49.53) (size 0.6) (drill 0.3) (layers "F.Cu" "B.Cu") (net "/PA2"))
 (segment (start 69.85 49.53) (end 80.01 49.53) (width 0.2) (layer "B.Cu") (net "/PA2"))
 (segment (start 82.55 36.83) (end 82.55 52.07) (width 0.2) (layer "F.Cu") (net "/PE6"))
 (segment (start 93.98 63.5) (end 99.06 63.5) (width 0.2) (layer "F.Cu") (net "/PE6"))
 (segment (start 82.55 52.07) (end 93.98 63.5) (width 0.2) (layer "F.Cu") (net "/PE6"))
 (segment (start 52.07 81.28) (end 62.19 71.16) (width 0.2) (layer "F.Cu") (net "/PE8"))
 (segment (start 62.19 71.16) (end 68.68 71.16) (width 0.2) (layer "F.Cu") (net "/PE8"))
 (segment (start 50.8 81.28) (end 52.07 81.28) (width 0.2) (layer "F.Cu") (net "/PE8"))
 (segment (start 81.18 71.16) (end 68.68 71.16) (width 0.2) (layer "F.Cu") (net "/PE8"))
 (segment (start 85.09 104.1) (end 81.18 104.1) (width 0.2) (layer "F.Cu") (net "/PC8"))
 (segment (start 85.13 104.1) (end 85.09 104.1) (width 0.2) (layer "F.Cu") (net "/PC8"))
 (segment (start 87.67 106.68) (end 85.09 104.1) (width 0.2) (layer "F.Cu") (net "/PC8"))
 (segment (start 99.06 106.68) (end 87.67 106.68) (width 0.2) (layer "F.Cu") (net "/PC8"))
 (segment (start 68.68 104.1) (end 81.18 104.1) (width 0.2) (layer "F.Cu") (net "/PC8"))
 (segment (start 99.06 104.14) (end 95.25 104.14) (width 0.2) (layer "F.Cu") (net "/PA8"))
 (segment (start 91.4 88.9) (end 91.4 93.88) (width 0.2) (layer "F.Cu") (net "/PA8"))
 (segment (start 91.4 100.29) (end 91.4 93.88) (width 0.2) (layer "F.Cu") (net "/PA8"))
 (segment (start 95.25 104.14) (end 91.4 100.29) (width 0.2) (layer "F.Cu") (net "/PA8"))
 (segment (start 91.4 81.38) (end 91.4 88.9) (width 0.2) (layer "F.Cu") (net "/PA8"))
 (segment (start 58.46 81.38) (end 58.46 93.88) (width 0.2) (layer "F.Cu") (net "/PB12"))
 (segment (start 50.8 93.98) (end 58.36 93.98) (width 0.2) (layer "F.Cu") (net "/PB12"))
 (segment (start 58.36 93.98) (end 58.46 93.88) (width 0.2) (layer "F.Cu") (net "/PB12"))
 (segment (start 99.06 53.34) (end 101.6 53.34) (width 0.2) (layer "F.Cu") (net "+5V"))
 (segment (start 101.6 53.34) (end 102.87 53.34) (width 0.2) (layer "F.Cu") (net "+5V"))
 (segment (start 104.14 104.14) (end 101.6 104.14) (width 0.2) (layer "F.Cu") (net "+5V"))
 (segment (start 102.87 53.34) (end 104.14 54.61) (width 0.2) (layer "F.Cu") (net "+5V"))
 (segment (start 104.14 54.61) (end 104.14 104.14) (width 0.2) (layer "F.Cu") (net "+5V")))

